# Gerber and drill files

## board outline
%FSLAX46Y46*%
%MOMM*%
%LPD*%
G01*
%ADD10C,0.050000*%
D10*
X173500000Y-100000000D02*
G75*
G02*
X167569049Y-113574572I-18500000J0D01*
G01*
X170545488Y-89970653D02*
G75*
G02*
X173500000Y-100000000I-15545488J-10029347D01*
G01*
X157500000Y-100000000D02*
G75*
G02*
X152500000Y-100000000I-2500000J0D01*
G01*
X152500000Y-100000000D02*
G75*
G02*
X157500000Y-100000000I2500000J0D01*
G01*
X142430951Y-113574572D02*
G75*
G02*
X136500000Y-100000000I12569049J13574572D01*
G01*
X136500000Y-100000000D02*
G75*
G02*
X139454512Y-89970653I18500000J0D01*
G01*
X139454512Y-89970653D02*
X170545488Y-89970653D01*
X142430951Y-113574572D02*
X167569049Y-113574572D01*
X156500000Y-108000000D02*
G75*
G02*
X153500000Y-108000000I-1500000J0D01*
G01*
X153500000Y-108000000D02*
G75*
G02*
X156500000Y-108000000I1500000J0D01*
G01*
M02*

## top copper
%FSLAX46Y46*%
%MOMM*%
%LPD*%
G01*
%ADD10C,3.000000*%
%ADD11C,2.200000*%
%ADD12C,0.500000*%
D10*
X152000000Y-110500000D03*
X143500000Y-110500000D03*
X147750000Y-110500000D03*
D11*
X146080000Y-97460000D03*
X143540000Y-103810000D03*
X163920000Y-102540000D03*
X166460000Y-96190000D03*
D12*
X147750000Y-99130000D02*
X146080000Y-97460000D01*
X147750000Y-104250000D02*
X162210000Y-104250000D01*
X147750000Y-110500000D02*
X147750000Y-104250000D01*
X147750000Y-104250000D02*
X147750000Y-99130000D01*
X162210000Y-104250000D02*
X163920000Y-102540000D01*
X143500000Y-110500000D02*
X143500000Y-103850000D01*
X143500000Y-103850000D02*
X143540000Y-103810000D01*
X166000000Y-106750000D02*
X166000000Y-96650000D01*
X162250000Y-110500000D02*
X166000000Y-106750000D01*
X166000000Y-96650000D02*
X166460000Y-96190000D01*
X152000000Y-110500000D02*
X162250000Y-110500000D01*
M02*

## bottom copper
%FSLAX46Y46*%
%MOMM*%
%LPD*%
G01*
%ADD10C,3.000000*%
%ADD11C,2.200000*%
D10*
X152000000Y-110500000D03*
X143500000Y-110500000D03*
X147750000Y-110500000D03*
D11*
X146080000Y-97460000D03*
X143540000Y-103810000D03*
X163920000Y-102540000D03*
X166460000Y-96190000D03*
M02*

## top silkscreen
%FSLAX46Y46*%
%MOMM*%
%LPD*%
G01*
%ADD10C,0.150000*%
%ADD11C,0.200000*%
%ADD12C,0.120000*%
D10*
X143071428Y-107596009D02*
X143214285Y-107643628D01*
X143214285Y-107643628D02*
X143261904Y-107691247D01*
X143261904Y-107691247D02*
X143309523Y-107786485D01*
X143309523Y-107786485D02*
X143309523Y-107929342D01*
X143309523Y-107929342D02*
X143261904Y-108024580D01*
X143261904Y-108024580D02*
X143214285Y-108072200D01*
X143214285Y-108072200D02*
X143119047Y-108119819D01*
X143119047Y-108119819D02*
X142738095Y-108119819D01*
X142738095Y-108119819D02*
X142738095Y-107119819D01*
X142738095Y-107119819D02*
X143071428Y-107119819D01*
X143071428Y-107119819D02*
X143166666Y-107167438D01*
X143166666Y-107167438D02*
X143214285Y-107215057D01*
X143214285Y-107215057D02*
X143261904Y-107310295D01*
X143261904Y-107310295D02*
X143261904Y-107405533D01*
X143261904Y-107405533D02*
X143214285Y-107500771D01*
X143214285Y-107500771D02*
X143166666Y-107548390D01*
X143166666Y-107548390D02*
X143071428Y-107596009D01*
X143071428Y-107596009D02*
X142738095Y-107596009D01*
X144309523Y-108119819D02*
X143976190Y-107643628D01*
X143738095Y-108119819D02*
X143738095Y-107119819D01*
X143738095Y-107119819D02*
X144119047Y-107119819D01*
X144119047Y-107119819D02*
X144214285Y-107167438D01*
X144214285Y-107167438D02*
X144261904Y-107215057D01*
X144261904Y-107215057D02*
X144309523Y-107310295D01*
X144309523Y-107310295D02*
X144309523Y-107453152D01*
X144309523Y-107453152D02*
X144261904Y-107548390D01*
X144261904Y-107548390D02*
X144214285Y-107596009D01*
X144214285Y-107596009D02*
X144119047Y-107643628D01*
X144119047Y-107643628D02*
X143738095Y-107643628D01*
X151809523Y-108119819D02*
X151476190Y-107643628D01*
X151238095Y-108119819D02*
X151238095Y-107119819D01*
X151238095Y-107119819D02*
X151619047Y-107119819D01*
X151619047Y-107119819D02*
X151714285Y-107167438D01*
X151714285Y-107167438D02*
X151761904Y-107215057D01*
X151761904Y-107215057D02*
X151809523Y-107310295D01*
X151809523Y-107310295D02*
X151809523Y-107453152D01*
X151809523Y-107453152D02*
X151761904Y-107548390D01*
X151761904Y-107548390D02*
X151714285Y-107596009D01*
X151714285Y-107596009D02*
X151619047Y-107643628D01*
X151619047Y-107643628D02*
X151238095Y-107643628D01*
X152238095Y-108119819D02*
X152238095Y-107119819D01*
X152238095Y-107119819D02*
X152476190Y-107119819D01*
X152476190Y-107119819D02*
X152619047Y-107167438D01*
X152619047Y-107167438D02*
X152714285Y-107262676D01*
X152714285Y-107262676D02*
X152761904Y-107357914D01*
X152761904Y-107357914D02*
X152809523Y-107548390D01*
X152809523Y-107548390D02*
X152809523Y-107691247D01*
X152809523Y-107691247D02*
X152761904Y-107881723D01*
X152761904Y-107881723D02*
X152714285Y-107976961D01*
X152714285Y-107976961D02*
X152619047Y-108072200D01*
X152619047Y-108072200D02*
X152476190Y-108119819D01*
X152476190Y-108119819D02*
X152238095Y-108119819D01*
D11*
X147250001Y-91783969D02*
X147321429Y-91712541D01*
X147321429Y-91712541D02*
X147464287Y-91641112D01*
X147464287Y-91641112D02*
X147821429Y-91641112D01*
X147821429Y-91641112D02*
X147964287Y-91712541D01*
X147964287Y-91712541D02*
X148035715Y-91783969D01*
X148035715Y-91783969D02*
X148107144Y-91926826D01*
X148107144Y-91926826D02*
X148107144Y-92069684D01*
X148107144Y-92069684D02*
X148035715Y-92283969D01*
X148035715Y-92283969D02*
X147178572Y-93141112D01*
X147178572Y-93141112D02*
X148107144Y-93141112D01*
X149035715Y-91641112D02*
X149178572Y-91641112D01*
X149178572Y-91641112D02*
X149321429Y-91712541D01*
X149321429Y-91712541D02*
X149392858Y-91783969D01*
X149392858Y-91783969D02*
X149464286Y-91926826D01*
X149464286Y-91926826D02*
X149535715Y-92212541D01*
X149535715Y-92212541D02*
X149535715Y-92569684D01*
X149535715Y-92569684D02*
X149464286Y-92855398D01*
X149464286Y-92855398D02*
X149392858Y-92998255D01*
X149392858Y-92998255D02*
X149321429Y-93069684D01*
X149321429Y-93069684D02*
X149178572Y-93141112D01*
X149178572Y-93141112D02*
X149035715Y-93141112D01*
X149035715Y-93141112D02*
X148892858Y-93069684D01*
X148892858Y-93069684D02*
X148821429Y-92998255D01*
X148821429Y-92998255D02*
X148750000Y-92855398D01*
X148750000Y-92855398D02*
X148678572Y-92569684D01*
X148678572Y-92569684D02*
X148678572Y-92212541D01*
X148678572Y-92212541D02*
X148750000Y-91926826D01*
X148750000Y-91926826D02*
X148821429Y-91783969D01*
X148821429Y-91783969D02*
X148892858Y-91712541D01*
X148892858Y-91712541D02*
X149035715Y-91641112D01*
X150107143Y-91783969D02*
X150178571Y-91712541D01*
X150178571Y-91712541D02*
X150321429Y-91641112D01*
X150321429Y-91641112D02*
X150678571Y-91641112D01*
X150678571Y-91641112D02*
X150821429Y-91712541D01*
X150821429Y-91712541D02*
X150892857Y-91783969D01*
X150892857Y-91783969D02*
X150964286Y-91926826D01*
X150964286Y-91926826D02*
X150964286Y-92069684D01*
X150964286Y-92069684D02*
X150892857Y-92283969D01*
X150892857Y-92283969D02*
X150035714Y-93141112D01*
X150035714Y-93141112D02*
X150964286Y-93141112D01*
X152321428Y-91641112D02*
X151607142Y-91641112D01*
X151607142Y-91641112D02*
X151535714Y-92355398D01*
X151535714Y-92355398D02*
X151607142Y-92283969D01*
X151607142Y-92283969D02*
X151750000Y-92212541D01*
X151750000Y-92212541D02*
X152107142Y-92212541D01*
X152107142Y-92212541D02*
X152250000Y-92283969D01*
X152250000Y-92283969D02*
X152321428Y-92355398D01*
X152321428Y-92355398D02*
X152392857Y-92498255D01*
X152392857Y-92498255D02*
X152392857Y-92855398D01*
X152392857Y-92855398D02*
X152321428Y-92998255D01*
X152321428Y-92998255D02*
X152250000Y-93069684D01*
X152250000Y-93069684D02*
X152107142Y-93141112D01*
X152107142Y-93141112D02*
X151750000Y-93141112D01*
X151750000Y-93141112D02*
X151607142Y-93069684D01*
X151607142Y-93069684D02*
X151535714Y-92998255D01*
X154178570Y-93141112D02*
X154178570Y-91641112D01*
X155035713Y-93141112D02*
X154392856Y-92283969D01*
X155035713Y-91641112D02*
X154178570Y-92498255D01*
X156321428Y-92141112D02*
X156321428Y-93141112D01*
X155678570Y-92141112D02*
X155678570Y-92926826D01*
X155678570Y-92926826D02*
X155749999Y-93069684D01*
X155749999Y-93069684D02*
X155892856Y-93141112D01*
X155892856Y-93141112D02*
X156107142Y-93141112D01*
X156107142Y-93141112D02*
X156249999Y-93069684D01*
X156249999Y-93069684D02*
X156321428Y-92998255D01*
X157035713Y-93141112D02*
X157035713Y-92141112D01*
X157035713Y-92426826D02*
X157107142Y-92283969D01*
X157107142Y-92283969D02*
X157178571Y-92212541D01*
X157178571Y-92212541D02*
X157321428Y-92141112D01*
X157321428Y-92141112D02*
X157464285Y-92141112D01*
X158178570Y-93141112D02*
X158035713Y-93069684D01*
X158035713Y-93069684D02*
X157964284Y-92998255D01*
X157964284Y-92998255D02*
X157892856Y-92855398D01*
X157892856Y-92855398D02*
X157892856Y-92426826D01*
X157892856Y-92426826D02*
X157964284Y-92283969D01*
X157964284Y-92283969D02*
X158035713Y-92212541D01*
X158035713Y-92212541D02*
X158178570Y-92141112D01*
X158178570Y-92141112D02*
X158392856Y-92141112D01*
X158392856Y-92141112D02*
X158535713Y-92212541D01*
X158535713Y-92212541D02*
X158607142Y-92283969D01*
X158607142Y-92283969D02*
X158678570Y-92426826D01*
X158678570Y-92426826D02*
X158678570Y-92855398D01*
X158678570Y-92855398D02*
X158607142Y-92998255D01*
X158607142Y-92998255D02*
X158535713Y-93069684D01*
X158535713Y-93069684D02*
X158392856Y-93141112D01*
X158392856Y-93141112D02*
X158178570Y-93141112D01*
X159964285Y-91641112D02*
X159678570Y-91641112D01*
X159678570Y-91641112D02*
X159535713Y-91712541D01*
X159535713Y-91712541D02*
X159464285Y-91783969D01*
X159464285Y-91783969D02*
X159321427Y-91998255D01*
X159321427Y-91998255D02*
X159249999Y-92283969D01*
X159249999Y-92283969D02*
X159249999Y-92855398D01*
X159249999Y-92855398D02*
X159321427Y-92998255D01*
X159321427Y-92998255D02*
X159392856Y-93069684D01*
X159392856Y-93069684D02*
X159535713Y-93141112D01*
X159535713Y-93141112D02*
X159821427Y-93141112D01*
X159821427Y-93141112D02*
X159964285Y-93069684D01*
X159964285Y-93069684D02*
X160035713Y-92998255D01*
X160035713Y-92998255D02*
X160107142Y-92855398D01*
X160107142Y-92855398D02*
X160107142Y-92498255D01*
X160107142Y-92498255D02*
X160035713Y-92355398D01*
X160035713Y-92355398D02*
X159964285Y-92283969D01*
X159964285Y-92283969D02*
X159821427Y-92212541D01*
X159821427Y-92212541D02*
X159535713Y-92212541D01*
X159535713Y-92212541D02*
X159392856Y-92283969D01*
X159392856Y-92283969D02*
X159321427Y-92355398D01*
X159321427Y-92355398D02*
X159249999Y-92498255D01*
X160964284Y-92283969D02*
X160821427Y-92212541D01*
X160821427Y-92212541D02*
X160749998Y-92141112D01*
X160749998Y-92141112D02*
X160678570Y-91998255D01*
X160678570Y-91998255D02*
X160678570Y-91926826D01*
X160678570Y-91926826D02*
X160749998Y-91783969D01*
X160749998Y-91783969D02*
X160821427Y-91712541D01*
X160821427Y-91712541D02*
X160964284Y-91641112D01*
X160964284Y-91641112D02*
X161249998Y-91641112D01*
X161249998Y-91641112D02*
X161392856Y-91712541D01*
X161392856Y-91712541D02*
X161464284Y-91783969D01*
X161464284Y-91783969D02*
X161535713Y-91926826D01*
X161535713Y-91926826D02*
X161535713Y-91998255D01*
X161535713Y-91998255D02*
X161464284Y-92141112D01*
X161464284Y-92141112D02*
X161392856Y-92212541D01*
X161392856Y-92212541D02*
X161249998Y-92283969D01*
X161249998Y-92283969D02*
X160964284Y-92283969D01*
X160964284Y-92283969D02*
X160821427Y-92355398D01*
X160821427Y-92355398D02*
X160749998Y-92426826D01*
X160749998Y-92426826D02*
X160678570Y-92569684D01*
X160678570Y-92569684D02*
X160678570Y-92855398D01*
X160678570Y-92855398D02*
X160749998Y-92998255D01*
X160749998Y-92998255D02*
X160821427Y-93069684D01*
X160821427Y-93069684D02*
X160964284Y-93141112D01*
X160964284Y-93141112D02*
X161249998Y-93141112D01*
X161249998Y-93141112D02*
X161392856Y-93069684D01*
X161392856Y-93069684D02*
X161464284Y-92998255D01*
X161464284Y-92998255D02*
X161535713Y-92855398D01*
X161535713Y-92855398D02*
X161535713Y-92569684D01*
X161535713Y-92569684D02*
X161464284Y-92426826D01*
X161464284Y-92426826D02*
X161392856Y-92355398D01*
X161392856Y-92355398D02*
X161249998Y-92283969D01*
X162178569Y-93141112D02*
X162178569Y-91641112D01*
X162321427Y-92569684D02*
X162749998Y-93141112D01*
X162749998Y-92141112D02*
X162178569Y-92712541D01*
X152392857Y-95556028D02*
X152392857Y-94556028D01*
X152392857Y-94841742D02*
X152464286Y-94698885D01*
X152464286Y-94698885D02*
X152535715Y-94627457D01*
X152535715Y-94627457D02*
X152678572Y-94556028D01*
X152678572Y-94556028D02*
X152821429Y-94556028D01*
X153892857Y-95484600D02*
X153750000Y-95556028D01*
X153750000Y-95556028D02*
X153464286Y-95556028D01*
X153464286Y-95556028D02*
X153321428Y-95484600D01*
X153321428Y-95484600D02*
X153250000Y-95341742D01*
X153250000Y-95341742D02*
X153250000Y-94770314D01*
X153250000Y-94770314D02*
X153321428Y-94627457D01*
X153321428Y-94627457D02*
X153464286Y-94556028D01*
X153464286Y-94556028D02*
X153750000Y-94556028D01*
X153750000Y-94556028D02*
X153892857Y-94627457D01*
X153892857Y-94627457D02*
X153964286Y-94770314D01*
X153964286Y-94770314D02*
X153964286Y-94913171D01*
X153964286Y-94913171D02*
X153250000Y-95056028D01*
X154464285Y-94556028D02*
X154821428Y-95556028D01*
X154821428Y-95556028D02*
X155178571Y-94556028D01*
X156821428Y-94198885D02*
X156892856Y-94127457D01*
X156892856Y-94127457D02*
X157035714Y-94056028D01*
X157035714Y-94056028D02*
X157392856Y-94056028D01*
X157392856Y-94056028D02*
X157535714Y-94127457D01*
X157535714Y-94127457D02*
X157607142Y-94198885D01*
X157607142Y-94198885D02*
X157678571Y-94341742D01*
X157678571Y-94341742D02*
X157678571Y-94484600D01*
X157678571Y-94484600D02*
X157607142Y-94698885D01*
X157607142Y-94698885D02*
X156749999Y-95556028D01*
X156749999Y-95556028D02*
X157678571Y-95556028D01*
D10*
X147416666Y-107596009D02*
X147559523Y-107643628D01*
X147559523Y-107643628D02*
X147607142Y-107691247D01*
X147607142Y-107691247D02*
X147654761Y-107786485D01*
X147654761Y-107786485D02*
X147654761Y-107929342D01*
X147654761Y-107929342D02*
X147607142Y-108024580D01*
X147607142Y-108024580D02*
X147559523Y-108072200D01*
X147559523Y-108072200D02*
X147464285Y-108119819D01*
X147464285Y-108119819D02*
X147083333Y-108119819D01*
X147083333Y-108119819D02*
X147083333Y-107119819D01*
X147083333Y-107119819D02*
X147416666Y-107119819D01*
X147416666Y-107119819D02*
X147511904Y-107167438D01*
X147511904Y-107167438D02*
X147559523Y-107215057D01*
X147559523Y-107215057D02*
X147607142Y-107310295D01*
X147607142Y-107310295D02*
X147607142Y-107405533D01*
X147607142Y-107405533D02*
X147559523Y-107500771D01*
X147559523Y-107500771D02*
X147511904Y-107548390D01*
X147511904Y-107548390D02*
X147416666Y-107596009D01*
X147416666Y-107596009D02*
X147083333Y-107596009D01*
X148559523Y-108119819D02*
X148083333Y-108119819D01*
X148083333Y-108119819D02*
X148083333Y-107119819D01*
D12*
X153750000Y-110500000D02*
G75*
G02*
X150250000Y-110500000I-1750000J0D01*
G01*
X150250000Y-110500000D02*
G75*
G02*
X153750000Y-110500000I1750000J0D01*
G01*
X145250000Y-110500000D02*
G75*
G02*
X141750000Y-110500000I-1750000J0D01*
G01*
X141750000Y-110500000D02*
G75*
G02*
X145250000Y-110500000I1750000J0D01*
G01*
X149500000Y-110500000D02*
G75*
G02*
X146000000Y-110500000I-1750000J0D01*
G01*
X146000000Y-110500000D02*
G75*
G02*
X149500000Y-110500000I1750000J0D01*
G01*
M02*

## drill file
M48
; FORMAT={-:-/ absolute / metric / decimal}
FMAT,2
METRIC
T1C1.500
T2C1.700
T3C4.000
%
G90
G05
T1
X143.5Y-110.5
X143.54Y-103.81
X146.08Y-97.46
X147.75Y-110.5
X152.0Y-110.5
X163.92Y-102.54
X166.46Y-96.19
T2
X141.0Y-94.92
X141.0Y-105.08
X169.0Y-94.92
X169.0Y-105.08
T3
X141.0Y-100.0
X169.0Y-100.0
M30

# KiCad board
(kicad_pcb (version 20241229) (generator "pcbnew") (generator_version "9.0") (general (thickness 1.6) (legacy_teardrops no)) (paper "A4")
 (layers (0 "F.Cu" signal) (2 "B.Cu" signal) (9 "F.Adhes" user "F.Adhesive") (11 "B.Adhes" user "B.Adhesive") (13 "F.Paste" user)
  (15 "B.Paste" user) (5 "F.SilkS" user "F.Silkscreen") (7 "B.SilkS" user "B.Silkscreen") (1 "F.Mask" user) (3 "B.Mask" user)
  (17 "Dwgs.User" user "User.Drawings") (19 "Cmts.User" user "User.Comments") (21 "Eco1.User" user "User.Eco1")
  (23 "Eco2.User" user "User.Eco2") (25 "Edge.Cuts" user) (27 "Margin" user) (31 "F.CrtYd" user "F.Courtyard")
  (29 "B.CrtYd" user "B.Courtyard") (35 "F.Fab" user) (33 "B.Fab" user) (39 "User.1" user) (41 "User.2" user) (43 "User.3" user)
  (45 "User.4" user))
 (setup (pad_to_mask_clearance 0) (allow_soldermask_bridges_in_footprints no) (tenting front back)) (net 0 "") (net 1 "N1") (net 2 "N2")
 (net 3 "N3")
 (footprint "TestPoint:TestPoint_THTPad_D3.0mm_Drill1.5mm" (layer "F.Cu") (at 152 110.5 90)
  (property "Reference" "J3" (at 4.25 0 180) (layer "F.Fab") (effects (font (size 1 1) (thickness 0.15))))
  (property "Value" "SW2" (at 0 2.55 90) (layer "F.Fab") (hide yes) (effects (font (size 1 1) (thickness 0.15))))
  (fp_circle (center 0 0) (end 0 1.75) (stroke (width 0.12) (type solid)) (fill no) (layer "F.SilkS"))
  (pad "1" thru_hole circle (at 0 0 90) (size 3 3) (drill 1.5) (layers "*.Cu" "*.Mask") (remove_unused_layers no) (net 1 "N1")))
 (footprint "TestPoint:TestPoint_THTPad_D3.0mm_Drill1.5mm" (layer "F.Cu") (at 143.5 110.5 90)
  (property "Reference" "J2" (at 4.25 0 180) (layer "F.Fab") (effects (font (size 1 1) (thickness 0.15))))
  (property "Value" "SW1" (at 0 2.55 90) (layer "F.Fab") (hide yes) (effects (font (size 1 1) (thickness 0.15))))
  (fp_circle (center 0 0) (end 0 1.75) (stroke (width 0.12) (type solid)) (fill no) (layer "F.SilkS"))
  (pad "1" thru_hole circle (at 0 0 90) (size 3 3) (drill 1.5) (layers "*.Cu" "*.Mask") (remove_unused_layers no) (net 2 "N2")))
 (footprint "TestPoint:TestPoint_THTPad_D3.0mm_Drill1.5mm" (layer "F.Cu") (at 147.75 110.5 90)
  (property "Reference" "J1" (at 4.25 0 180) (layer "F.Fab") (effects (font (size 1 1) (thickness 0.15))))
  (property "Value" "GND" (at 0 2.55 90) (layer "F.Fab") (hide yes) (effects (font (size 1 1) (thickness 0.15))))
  (fp_circle (center 0 0) (end 0 1.75) (stroke (width 0.12) (type solid)) (fill no) (layer "F.SilkS"))
  (pad "1" thru_hole circle (at 0 0 90) (size 3 3) (drill 1.5) (layers "*.Cu" "*.Mask") (remove_unused_layers no) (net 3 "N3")))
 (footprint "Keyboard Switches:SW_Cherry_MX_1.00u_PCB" (layer "B.Cu") (at 146.08 97.46 90)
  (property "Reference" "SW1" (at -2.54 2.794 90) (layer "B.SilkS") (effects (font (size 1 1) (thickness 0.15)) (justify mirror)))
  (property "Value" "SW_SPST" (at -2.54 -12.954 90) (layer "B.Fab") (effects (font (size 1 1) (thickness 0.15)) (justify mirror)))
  (pad "" np_thru_hole circle (at -7.62 -5.08 90) (size 1.7 1.7) (drill 1.7) (layers "*.Cu" "*.Mask"))
  (pad "" np_thru_hole circle (at -2.54 -5.08 90) (size 4 4) (drill 4) (layers "*.Cu" "*.Mask"))
  (pad "" np_thru_hole circle (at 2.54 -5.08 90) (size 1.7 1.7) (drill 1.7) (layers "*.Cu" "*.Mask"))
  (pad "1" thru_hole circle (at 0 0 90) (size 2.2 2.2) (drill 1.5) (layers "*.Cu" "*.Mask") (remove_unused_layers no) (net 3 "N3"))
  (pad "2" thru_hole circle (at -6.35 -2.54 90) (size 2.2 2.2) (drill 1.5) (layers "*.Cu" "*.Mask") (remove_unused_layers no) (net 2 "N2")))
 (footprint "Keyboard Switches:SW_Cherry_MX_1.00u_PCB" (layer "B.Cu") (at 163.92 102.54 -90)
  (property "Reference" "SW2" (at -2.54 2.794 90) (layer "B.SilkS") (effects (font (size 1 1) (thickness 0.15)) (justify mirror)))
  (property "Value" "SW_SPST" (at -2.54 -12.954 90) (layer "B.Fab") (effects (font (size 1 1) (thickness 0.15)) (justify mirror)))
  (pad "" np_thru_hole circle (at -7.62 -5.08 270) (size 1.7 1.7) (drill 1.7) (layers "*.Cu" "*.Mask"))
  (pad "" np_thru_hole circle (at -2.54 -5.08 270) (size 4 4) (drill 4) (layers "*.Cu" "*.Mask"))
  (pad "" np_thru_hole circle (at 2.54 -5.08 270) (size 1.7 1.7) (drill 1.7) (layers "*.Cu" "*.Mask"))
  (pad "1" thru_hole circle (at 0 0 270) (size 2.2 2.2) (drill 1.5) (layers "*.Cu" "*.Mask") (remove_unused_layers no) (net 3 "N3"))
  (pad "2" thru_hole circle (at -6.35 -2.54 270) (size 2.2 2.2) (drill 1.5) (layers "*.Cu" "*.Mask") (remove_unused_layers no) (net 1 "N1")))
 (gr_arc (start 173.5 100) (mid 171.952543 107.406841) (end 167.569049 113.574572) (stroke (width 0.05) (type default)) (layer "Edge.Cuts"))
 (gr_arc (start 170.545488 89.970653) (mid 172.746007 94.772263) (end 173.5 100) (stroke (width 0.05) (type default)) (layer "Edge.Cuts"))
 (gr_circle (center 155 100) (end 157.5 100) (stroke (width 0.05) (type default)) (fill no) (layer "Edge.Cuts"))
 (gr_arc (start 142.430951 113.574572) (mid 138.047457 107.406841) (end 136.5 100) (stroke (width 0.05) (type default)) (layer "Edge.Cuts"))
 (gr_arc (start 136.5 100) (mid 137.253993 94.772263) (end 139.454512 89.970653) (stroke (width 0.05) (type default)) (layer "Edge.Cuts"))
 (gr_line (start 139.454512 89.970653) (end 170.545488 89.970653) (stroke (width 0.05) (type default)) (layer "Edge.Cuts"))
 (gr_line (start 142.430951 113.574572) (end 167.569049 113.574572) (stroke (width 0.05) (type default)) (layer "Edge.Cuts"))
 (gr_circle (center 155 108) (end 156.5 108) (stroke (width 0.05) (type solid)) (fill no) (layer "Edge.Cuts"))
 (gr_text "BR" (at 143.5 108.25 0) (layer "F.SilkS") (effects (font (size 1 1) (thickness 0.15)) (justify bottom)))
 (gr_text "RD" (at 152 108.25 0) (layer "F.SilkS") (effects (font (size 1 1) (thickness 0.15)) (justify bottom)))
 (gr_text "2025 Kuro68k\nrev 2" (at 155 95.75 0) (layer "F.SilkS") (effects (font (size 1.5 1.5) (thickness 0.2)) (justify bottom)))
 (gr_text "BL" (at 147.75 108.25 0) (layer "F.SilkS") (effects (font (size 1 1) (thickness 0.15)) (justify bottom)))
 (segment (start 147.75 99.13) (end 146.08 97.46) (width 0.5) (layer "F.Cu") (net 3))
 (segment (start 147.75 104.25) (end 162.21 104.25) (width 0.5) (layer "F.Cu") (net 3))
 (segment (start 147.75 110.5) (end 147.75 104.25) (width 0.5) (layer "F.Cu") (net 3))
 (segment (start 147.75 104.25) (end 147.75 99.13) (width 0.5) (layer "F.Cu") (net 3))
 (segment (start 162.21 104.25) (end 163.92 102.54) (width 0.5) (layer "F.Cu") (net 3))
 (segment (start 143.5 110.5) (end 143.5 103.85) (width 0.5) (layer "F.Cu") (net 2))
 (segment (start 143.5 103.85) (end 143.54 103.81) (width 0.5) (layer "F.Cu") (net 2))
 (segment (start 166 106.75) (end 166 96.65) (width 0.5) (layer "F.Cu") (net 1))
 (segment (start 162.25 110.5) (end 166 106.75) (width 0.5) (layer "F.Cu") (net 1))
 (segment (start 166 96.65) (end 166.46 96.19) (width 0.5) (layer "F.Cu") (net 1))
 (segment (start 152 110.5) (end 162.25 110.5) (width 0.5) (layer "F.Cu") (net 1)))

